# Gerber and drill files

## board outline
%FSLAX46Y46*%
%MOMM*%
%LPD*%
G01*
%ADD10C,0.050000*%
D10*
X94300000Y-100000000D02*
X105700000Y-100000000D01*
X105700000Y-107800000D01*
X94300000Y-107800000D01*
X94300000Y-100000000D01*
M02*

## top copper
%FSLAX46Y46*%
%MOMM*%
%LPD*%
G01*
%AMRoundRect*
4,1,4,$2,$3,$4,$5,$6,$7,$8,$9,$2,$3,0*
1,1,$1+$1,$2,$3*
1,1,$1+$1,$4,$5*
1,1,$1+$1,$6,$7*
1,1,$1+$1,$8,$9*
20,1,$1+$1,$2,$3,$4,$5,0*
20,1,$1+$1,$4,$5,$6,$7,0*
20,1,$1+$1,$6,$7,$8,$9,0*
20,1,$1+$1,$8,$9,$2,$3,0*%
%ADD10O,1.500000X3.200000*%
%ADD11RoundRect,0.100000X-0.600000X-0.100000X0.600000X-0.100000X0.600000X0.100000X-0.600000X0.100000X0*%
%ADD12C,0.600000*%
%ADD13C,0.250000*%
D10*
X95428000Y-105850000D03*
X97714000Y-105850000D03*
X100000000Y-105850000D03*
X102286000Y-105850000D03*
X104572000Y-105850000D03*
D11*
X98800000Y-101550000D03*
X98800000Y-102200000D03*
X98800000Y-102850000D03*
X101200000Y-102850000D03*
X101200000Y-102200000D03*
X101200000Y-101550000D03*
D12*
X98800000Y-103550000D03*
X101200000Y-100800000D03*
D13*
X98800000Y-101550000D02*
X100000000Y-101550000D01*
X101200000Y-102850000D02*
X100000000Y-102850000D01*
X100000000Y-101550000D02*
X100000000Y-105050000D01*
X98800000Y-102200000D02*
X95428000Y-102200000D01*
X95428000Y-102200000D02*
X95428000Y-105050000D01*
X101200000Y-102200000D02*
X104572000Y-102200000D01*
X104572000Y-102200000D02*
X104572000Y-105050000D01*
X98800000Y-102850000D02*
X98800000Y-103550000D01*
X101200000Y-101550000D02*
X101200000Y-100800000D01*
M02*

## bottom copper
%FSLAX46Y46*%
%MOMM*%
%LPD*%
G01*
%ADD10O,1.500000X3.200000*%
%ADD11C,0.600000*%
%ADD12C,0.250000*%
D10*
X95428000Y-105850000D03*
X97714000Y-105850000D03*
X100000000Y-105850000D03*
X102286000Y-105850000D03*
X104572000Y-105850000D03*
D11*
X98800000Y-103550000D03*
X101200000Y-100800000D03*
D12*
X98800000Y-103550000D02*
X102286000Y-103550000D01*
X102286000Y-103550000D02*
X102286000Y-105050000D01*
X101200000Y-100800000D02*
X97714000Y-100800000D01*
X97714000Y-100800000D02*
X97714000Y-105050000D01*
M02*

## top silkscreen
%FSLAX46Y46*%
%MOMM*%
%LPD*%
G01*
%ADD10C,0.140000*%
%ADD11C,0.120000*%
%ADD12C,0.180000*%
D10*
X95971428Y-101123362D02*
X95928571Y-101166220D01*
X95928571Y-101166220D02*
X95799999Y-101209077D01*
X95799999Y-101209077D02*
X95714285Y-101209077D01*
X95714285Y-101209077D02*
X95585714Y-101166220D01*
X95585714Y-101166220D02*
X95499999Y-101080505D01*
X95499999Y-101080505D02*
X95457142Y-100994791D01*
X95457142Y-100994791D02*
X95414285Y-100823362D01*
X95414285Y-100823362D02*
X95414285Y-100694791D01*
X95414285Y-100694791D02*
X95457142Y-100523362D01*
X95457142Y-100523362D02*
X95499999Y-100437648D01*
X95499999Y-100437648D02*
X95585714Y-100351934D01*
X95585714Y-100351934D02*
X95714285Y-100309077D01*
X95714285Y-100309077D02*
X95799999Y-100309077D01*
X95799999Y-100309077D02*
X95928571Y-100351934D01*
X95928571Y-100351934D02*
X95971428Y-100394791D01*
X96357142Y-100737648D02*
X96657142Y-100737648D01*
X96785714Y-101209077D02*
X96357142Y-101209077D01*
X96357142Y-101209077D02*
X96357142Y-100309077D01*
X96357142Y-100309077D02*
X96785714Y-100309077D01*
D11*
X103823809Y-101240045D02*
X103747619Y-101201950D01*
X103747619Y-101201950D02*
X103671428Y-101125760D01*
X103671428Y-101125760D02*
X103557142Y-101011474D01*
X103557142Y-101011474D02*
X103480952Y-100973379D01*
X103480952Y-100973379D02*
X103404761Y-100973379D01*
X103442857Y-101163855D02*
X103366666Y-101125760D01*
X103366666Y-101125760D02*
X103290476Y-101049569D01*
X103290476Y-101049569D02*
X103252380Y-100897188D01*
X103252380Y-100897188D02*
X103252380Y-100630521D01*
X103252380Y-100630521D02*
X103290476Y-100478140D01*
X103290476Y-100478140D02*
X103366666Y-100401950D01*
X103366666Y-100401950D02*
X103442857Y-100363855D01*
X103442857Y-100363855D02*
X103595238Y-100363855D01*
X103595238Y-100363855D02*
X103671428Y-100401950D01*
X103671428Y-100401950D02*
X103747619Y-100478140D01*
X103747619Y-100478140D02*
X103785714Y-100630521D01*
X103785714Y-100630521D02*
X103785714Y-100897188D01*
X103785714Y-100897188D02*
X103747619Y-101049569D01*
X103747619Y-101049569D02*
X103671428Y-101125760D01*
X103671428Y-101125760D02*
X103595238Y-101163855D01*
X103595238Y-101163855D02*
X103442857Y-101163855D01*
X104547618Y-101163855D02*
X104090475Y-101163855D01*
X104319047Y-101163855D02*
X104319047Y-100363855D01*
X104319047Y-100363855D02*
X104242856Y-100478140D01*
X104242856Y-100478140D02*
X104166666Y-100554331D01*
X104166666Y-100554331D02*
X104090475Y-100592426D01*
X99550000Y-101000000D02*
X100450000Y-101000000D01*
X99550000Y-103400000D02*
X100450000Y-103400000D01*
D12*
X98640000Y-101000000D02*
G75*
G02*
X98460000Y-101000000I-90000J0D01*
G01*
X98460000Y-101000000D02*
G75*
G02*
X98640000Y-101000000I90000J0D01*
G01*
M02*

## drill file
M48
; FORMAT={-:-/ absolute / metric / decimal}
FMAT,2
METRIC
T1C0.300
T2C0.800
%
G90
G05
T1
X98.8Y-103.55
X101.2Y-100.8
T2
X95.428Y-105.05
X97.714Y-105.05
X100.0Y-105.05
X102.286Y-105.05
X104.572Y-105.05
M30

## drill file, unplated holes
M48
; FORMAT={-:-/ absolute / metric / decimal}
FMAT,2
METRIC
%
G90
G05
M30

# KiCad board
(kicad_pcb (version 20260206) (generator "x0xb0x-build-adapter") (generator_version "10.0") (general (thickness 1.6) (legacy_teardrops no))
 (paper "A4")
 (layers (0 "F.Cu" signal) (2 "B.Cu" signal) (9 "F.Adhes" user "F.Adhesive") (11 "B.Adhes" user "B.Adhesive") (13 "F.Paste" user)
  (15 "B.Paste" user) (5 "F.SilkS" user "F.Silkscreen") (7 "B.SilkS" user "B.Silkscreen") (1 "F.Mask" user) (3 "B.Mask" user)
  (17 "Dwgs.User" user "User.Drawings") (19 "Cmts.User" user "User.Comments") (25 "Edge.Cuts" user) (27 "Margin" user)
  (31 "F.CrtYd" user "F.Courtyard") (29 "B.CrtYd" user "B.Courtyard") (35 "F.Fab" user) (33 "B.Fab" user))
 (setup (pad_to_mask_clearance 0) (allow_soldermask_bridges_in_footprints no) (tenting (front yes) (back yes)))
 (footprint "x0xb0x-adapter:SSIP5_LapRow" (layer "F.Cu") (at 100.0 105.05)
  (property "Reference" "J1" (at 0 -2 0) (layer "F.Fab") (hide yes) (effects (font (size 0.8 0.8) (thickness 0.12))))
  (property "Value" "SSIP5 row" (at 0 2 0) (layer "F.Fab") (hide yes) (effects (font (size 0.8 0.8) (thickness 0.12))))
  (pad "1" thru_hole oval (at -4.572 0) (size 1.5 3.2) (drill 0.8 (offset 0 0.8)) (layers "*.Cu" "*.Mask") (remove_unused_layers no)
   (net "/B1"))
  (pad "2" thru_hole oval (at -2.286 0) (size 1.5 3.2) (drill 0.8 (offset 0 0.8)) (layers "*.Cu" "*.Mask") (remove_unused_layers no)
   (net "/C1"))
  (pad "3" thru_hole oval (at 0.000 0) (size 1.5 3.2) (drill 0.8 (offset 0 0.8)) (layers "*.Cu" "*.Mask") (remove_unused_layers no)
   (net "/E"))
  (pad "4" thru_hole oval (at 2.286 0) (size 1.5 3.2) (drill 0.8 (offset 0 0.8)) (layers "*.Cu" "*.Mask") (remove_unused_layers no)
   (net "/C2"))
  (pad "5" thru_hole oval (at 4.572 0) (size 1.5 3.2) (drill 0.8 (offset 0 0.8)) (layers "*.Cu" "*.Mask") (remove_unused_layers no)
   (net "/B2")))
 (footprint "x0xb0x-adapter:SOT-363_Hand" (layer "F.Cu") (at 100.0 102.2)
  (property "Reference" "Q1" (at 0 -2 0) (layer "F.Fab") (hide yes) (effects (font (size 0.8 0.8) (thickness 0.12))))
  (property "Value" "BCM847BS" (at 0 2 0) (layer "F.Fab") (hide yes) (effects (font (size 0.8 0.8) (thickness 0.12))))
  (fp_line (start -0.45 -1.2) (end 0.45 -1.2) (stroke (width 0.12) (type solid)) (layer "F.SilkS"))
  (fp_line (start -0.45 1.2) (end 0.45 1.2) (stroke (width 0.12) (type solid)) (layer "F.SilkS"))
  (fp_circle (center -1.45 -1.2) (end -1.33 -1.2) (stroke (width 0.12) (type solid)) (fill yes) (layer "F.SilkS"))
  (pad "1" smd roundrect (at -1.2 -0.65) (size 1.4 0.4) (layers "F.Cu" "F.Mask" "F.Paste") (roundrect_rratio 0.25) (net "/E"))
  (pad "2" smd roundrect (at -1.2 0) (size 1.4 0.4) (layers "F.Cu" "F.Mask" "F.Paste") (roundrect_rratio 0.25) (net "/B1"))
  (pad "3" smd roundrect (at -1.2 0.65) (size 1.4 0.4) (layers "F.Cu" "F.Mask" "F.Paste") (roundrect_rratio 0.25) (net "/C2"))
  (pad "4" smd roundrect (at 1.2 0.65) (size 1.4 0.4) (layers "F.Cu" "F.Mask" "F.Paste") (roundrect_rratio 0.25) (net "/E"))
  (pad "5" smd roundrect (at 1.2 0) (size 1.4 0.4) (layers "F.Cu" "F.Mask" "F.Paste") (roundrect_rratio 0.25) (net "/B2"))
  (pad "6" smd roundrect (at 1.2 -0.65) (size 1.4 0.4) (layers "F.Cu" "F.Mask" "F.Paste") (roundrect_rratio 0.25) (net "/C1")))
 (segment (start 98.8 101.55) (end 100.0 101.55) (width 0.25) (layer "F.Cu") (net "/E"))
 (segment (start 101.2 102.85) (end 100.0 102.85) (width 0.25) (layer "F.Cu") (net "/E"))
 (segment (start 100.0 101.55) (end 100.0 105.05) (width 0.25) (layer "F.Cu") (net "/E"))
 (segment (start 98.8 102.2) (end 95.428 102.2) (width 0.25) (layer "F.Cu") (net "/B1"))
 (segment (start 95.428 102.2) (end 95.428 105.05) (width 0.25) (layer "F.Cu") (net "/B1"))
 (segment (start 101.2 102.2) (end 104.572 102.2) (width 0.25) (layer "F.Cu") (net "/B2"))
 (segment (start 104.572 102.2) (end 104.572 105.05) (width 0.25) (layer "F.Cu") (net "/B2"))
 (segment (start 98.8 102.85) (end 98.8 103.55) (width 0.25) (layer "F.Cu") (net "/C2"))
 (segment (start 98.8 103.55) (end 102.286 103.55) (width 0.25) (layer "B.Cu") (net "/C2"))
 (segment (start 102.286 103.55) (end 102.286 105.05) (width 0.25) (layer "B.Cu") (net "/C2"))
 (segment (start 101.2 101.55) (end 101.2 100.8) (width 0.25) (layer "F.Cu") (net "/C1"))
 (segment (start 101.2 100.8) (end 97.714 100.8) (width 0.25) (layer "B.Cu") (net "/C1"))
 (segment (start 97.714 100.8) (end 97.714 105.05) (width 0.25) (layer "B.Cu") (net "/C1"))
 (via (at 98.8 103.55) (size 0.6) (drill 0.3) (layers "F.Cu" "B.Cu") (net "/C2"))
 (via (at 101.2 100.8) (size 0.6) (drill 0.3) (layers "F.Cu" "B.Cu") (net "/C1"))
 (gr_rect (start 94.3 100.0) (end 105.7 107.8) (stroke (width 0.05) (type default)) (fill no) (layer "Edge.Cuts"))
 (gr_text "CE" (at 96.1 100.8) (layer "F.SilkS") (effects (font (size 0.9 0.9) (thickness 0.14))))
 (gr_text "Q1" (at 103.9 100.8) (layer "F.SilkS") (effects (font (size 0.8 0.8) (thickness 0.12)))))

